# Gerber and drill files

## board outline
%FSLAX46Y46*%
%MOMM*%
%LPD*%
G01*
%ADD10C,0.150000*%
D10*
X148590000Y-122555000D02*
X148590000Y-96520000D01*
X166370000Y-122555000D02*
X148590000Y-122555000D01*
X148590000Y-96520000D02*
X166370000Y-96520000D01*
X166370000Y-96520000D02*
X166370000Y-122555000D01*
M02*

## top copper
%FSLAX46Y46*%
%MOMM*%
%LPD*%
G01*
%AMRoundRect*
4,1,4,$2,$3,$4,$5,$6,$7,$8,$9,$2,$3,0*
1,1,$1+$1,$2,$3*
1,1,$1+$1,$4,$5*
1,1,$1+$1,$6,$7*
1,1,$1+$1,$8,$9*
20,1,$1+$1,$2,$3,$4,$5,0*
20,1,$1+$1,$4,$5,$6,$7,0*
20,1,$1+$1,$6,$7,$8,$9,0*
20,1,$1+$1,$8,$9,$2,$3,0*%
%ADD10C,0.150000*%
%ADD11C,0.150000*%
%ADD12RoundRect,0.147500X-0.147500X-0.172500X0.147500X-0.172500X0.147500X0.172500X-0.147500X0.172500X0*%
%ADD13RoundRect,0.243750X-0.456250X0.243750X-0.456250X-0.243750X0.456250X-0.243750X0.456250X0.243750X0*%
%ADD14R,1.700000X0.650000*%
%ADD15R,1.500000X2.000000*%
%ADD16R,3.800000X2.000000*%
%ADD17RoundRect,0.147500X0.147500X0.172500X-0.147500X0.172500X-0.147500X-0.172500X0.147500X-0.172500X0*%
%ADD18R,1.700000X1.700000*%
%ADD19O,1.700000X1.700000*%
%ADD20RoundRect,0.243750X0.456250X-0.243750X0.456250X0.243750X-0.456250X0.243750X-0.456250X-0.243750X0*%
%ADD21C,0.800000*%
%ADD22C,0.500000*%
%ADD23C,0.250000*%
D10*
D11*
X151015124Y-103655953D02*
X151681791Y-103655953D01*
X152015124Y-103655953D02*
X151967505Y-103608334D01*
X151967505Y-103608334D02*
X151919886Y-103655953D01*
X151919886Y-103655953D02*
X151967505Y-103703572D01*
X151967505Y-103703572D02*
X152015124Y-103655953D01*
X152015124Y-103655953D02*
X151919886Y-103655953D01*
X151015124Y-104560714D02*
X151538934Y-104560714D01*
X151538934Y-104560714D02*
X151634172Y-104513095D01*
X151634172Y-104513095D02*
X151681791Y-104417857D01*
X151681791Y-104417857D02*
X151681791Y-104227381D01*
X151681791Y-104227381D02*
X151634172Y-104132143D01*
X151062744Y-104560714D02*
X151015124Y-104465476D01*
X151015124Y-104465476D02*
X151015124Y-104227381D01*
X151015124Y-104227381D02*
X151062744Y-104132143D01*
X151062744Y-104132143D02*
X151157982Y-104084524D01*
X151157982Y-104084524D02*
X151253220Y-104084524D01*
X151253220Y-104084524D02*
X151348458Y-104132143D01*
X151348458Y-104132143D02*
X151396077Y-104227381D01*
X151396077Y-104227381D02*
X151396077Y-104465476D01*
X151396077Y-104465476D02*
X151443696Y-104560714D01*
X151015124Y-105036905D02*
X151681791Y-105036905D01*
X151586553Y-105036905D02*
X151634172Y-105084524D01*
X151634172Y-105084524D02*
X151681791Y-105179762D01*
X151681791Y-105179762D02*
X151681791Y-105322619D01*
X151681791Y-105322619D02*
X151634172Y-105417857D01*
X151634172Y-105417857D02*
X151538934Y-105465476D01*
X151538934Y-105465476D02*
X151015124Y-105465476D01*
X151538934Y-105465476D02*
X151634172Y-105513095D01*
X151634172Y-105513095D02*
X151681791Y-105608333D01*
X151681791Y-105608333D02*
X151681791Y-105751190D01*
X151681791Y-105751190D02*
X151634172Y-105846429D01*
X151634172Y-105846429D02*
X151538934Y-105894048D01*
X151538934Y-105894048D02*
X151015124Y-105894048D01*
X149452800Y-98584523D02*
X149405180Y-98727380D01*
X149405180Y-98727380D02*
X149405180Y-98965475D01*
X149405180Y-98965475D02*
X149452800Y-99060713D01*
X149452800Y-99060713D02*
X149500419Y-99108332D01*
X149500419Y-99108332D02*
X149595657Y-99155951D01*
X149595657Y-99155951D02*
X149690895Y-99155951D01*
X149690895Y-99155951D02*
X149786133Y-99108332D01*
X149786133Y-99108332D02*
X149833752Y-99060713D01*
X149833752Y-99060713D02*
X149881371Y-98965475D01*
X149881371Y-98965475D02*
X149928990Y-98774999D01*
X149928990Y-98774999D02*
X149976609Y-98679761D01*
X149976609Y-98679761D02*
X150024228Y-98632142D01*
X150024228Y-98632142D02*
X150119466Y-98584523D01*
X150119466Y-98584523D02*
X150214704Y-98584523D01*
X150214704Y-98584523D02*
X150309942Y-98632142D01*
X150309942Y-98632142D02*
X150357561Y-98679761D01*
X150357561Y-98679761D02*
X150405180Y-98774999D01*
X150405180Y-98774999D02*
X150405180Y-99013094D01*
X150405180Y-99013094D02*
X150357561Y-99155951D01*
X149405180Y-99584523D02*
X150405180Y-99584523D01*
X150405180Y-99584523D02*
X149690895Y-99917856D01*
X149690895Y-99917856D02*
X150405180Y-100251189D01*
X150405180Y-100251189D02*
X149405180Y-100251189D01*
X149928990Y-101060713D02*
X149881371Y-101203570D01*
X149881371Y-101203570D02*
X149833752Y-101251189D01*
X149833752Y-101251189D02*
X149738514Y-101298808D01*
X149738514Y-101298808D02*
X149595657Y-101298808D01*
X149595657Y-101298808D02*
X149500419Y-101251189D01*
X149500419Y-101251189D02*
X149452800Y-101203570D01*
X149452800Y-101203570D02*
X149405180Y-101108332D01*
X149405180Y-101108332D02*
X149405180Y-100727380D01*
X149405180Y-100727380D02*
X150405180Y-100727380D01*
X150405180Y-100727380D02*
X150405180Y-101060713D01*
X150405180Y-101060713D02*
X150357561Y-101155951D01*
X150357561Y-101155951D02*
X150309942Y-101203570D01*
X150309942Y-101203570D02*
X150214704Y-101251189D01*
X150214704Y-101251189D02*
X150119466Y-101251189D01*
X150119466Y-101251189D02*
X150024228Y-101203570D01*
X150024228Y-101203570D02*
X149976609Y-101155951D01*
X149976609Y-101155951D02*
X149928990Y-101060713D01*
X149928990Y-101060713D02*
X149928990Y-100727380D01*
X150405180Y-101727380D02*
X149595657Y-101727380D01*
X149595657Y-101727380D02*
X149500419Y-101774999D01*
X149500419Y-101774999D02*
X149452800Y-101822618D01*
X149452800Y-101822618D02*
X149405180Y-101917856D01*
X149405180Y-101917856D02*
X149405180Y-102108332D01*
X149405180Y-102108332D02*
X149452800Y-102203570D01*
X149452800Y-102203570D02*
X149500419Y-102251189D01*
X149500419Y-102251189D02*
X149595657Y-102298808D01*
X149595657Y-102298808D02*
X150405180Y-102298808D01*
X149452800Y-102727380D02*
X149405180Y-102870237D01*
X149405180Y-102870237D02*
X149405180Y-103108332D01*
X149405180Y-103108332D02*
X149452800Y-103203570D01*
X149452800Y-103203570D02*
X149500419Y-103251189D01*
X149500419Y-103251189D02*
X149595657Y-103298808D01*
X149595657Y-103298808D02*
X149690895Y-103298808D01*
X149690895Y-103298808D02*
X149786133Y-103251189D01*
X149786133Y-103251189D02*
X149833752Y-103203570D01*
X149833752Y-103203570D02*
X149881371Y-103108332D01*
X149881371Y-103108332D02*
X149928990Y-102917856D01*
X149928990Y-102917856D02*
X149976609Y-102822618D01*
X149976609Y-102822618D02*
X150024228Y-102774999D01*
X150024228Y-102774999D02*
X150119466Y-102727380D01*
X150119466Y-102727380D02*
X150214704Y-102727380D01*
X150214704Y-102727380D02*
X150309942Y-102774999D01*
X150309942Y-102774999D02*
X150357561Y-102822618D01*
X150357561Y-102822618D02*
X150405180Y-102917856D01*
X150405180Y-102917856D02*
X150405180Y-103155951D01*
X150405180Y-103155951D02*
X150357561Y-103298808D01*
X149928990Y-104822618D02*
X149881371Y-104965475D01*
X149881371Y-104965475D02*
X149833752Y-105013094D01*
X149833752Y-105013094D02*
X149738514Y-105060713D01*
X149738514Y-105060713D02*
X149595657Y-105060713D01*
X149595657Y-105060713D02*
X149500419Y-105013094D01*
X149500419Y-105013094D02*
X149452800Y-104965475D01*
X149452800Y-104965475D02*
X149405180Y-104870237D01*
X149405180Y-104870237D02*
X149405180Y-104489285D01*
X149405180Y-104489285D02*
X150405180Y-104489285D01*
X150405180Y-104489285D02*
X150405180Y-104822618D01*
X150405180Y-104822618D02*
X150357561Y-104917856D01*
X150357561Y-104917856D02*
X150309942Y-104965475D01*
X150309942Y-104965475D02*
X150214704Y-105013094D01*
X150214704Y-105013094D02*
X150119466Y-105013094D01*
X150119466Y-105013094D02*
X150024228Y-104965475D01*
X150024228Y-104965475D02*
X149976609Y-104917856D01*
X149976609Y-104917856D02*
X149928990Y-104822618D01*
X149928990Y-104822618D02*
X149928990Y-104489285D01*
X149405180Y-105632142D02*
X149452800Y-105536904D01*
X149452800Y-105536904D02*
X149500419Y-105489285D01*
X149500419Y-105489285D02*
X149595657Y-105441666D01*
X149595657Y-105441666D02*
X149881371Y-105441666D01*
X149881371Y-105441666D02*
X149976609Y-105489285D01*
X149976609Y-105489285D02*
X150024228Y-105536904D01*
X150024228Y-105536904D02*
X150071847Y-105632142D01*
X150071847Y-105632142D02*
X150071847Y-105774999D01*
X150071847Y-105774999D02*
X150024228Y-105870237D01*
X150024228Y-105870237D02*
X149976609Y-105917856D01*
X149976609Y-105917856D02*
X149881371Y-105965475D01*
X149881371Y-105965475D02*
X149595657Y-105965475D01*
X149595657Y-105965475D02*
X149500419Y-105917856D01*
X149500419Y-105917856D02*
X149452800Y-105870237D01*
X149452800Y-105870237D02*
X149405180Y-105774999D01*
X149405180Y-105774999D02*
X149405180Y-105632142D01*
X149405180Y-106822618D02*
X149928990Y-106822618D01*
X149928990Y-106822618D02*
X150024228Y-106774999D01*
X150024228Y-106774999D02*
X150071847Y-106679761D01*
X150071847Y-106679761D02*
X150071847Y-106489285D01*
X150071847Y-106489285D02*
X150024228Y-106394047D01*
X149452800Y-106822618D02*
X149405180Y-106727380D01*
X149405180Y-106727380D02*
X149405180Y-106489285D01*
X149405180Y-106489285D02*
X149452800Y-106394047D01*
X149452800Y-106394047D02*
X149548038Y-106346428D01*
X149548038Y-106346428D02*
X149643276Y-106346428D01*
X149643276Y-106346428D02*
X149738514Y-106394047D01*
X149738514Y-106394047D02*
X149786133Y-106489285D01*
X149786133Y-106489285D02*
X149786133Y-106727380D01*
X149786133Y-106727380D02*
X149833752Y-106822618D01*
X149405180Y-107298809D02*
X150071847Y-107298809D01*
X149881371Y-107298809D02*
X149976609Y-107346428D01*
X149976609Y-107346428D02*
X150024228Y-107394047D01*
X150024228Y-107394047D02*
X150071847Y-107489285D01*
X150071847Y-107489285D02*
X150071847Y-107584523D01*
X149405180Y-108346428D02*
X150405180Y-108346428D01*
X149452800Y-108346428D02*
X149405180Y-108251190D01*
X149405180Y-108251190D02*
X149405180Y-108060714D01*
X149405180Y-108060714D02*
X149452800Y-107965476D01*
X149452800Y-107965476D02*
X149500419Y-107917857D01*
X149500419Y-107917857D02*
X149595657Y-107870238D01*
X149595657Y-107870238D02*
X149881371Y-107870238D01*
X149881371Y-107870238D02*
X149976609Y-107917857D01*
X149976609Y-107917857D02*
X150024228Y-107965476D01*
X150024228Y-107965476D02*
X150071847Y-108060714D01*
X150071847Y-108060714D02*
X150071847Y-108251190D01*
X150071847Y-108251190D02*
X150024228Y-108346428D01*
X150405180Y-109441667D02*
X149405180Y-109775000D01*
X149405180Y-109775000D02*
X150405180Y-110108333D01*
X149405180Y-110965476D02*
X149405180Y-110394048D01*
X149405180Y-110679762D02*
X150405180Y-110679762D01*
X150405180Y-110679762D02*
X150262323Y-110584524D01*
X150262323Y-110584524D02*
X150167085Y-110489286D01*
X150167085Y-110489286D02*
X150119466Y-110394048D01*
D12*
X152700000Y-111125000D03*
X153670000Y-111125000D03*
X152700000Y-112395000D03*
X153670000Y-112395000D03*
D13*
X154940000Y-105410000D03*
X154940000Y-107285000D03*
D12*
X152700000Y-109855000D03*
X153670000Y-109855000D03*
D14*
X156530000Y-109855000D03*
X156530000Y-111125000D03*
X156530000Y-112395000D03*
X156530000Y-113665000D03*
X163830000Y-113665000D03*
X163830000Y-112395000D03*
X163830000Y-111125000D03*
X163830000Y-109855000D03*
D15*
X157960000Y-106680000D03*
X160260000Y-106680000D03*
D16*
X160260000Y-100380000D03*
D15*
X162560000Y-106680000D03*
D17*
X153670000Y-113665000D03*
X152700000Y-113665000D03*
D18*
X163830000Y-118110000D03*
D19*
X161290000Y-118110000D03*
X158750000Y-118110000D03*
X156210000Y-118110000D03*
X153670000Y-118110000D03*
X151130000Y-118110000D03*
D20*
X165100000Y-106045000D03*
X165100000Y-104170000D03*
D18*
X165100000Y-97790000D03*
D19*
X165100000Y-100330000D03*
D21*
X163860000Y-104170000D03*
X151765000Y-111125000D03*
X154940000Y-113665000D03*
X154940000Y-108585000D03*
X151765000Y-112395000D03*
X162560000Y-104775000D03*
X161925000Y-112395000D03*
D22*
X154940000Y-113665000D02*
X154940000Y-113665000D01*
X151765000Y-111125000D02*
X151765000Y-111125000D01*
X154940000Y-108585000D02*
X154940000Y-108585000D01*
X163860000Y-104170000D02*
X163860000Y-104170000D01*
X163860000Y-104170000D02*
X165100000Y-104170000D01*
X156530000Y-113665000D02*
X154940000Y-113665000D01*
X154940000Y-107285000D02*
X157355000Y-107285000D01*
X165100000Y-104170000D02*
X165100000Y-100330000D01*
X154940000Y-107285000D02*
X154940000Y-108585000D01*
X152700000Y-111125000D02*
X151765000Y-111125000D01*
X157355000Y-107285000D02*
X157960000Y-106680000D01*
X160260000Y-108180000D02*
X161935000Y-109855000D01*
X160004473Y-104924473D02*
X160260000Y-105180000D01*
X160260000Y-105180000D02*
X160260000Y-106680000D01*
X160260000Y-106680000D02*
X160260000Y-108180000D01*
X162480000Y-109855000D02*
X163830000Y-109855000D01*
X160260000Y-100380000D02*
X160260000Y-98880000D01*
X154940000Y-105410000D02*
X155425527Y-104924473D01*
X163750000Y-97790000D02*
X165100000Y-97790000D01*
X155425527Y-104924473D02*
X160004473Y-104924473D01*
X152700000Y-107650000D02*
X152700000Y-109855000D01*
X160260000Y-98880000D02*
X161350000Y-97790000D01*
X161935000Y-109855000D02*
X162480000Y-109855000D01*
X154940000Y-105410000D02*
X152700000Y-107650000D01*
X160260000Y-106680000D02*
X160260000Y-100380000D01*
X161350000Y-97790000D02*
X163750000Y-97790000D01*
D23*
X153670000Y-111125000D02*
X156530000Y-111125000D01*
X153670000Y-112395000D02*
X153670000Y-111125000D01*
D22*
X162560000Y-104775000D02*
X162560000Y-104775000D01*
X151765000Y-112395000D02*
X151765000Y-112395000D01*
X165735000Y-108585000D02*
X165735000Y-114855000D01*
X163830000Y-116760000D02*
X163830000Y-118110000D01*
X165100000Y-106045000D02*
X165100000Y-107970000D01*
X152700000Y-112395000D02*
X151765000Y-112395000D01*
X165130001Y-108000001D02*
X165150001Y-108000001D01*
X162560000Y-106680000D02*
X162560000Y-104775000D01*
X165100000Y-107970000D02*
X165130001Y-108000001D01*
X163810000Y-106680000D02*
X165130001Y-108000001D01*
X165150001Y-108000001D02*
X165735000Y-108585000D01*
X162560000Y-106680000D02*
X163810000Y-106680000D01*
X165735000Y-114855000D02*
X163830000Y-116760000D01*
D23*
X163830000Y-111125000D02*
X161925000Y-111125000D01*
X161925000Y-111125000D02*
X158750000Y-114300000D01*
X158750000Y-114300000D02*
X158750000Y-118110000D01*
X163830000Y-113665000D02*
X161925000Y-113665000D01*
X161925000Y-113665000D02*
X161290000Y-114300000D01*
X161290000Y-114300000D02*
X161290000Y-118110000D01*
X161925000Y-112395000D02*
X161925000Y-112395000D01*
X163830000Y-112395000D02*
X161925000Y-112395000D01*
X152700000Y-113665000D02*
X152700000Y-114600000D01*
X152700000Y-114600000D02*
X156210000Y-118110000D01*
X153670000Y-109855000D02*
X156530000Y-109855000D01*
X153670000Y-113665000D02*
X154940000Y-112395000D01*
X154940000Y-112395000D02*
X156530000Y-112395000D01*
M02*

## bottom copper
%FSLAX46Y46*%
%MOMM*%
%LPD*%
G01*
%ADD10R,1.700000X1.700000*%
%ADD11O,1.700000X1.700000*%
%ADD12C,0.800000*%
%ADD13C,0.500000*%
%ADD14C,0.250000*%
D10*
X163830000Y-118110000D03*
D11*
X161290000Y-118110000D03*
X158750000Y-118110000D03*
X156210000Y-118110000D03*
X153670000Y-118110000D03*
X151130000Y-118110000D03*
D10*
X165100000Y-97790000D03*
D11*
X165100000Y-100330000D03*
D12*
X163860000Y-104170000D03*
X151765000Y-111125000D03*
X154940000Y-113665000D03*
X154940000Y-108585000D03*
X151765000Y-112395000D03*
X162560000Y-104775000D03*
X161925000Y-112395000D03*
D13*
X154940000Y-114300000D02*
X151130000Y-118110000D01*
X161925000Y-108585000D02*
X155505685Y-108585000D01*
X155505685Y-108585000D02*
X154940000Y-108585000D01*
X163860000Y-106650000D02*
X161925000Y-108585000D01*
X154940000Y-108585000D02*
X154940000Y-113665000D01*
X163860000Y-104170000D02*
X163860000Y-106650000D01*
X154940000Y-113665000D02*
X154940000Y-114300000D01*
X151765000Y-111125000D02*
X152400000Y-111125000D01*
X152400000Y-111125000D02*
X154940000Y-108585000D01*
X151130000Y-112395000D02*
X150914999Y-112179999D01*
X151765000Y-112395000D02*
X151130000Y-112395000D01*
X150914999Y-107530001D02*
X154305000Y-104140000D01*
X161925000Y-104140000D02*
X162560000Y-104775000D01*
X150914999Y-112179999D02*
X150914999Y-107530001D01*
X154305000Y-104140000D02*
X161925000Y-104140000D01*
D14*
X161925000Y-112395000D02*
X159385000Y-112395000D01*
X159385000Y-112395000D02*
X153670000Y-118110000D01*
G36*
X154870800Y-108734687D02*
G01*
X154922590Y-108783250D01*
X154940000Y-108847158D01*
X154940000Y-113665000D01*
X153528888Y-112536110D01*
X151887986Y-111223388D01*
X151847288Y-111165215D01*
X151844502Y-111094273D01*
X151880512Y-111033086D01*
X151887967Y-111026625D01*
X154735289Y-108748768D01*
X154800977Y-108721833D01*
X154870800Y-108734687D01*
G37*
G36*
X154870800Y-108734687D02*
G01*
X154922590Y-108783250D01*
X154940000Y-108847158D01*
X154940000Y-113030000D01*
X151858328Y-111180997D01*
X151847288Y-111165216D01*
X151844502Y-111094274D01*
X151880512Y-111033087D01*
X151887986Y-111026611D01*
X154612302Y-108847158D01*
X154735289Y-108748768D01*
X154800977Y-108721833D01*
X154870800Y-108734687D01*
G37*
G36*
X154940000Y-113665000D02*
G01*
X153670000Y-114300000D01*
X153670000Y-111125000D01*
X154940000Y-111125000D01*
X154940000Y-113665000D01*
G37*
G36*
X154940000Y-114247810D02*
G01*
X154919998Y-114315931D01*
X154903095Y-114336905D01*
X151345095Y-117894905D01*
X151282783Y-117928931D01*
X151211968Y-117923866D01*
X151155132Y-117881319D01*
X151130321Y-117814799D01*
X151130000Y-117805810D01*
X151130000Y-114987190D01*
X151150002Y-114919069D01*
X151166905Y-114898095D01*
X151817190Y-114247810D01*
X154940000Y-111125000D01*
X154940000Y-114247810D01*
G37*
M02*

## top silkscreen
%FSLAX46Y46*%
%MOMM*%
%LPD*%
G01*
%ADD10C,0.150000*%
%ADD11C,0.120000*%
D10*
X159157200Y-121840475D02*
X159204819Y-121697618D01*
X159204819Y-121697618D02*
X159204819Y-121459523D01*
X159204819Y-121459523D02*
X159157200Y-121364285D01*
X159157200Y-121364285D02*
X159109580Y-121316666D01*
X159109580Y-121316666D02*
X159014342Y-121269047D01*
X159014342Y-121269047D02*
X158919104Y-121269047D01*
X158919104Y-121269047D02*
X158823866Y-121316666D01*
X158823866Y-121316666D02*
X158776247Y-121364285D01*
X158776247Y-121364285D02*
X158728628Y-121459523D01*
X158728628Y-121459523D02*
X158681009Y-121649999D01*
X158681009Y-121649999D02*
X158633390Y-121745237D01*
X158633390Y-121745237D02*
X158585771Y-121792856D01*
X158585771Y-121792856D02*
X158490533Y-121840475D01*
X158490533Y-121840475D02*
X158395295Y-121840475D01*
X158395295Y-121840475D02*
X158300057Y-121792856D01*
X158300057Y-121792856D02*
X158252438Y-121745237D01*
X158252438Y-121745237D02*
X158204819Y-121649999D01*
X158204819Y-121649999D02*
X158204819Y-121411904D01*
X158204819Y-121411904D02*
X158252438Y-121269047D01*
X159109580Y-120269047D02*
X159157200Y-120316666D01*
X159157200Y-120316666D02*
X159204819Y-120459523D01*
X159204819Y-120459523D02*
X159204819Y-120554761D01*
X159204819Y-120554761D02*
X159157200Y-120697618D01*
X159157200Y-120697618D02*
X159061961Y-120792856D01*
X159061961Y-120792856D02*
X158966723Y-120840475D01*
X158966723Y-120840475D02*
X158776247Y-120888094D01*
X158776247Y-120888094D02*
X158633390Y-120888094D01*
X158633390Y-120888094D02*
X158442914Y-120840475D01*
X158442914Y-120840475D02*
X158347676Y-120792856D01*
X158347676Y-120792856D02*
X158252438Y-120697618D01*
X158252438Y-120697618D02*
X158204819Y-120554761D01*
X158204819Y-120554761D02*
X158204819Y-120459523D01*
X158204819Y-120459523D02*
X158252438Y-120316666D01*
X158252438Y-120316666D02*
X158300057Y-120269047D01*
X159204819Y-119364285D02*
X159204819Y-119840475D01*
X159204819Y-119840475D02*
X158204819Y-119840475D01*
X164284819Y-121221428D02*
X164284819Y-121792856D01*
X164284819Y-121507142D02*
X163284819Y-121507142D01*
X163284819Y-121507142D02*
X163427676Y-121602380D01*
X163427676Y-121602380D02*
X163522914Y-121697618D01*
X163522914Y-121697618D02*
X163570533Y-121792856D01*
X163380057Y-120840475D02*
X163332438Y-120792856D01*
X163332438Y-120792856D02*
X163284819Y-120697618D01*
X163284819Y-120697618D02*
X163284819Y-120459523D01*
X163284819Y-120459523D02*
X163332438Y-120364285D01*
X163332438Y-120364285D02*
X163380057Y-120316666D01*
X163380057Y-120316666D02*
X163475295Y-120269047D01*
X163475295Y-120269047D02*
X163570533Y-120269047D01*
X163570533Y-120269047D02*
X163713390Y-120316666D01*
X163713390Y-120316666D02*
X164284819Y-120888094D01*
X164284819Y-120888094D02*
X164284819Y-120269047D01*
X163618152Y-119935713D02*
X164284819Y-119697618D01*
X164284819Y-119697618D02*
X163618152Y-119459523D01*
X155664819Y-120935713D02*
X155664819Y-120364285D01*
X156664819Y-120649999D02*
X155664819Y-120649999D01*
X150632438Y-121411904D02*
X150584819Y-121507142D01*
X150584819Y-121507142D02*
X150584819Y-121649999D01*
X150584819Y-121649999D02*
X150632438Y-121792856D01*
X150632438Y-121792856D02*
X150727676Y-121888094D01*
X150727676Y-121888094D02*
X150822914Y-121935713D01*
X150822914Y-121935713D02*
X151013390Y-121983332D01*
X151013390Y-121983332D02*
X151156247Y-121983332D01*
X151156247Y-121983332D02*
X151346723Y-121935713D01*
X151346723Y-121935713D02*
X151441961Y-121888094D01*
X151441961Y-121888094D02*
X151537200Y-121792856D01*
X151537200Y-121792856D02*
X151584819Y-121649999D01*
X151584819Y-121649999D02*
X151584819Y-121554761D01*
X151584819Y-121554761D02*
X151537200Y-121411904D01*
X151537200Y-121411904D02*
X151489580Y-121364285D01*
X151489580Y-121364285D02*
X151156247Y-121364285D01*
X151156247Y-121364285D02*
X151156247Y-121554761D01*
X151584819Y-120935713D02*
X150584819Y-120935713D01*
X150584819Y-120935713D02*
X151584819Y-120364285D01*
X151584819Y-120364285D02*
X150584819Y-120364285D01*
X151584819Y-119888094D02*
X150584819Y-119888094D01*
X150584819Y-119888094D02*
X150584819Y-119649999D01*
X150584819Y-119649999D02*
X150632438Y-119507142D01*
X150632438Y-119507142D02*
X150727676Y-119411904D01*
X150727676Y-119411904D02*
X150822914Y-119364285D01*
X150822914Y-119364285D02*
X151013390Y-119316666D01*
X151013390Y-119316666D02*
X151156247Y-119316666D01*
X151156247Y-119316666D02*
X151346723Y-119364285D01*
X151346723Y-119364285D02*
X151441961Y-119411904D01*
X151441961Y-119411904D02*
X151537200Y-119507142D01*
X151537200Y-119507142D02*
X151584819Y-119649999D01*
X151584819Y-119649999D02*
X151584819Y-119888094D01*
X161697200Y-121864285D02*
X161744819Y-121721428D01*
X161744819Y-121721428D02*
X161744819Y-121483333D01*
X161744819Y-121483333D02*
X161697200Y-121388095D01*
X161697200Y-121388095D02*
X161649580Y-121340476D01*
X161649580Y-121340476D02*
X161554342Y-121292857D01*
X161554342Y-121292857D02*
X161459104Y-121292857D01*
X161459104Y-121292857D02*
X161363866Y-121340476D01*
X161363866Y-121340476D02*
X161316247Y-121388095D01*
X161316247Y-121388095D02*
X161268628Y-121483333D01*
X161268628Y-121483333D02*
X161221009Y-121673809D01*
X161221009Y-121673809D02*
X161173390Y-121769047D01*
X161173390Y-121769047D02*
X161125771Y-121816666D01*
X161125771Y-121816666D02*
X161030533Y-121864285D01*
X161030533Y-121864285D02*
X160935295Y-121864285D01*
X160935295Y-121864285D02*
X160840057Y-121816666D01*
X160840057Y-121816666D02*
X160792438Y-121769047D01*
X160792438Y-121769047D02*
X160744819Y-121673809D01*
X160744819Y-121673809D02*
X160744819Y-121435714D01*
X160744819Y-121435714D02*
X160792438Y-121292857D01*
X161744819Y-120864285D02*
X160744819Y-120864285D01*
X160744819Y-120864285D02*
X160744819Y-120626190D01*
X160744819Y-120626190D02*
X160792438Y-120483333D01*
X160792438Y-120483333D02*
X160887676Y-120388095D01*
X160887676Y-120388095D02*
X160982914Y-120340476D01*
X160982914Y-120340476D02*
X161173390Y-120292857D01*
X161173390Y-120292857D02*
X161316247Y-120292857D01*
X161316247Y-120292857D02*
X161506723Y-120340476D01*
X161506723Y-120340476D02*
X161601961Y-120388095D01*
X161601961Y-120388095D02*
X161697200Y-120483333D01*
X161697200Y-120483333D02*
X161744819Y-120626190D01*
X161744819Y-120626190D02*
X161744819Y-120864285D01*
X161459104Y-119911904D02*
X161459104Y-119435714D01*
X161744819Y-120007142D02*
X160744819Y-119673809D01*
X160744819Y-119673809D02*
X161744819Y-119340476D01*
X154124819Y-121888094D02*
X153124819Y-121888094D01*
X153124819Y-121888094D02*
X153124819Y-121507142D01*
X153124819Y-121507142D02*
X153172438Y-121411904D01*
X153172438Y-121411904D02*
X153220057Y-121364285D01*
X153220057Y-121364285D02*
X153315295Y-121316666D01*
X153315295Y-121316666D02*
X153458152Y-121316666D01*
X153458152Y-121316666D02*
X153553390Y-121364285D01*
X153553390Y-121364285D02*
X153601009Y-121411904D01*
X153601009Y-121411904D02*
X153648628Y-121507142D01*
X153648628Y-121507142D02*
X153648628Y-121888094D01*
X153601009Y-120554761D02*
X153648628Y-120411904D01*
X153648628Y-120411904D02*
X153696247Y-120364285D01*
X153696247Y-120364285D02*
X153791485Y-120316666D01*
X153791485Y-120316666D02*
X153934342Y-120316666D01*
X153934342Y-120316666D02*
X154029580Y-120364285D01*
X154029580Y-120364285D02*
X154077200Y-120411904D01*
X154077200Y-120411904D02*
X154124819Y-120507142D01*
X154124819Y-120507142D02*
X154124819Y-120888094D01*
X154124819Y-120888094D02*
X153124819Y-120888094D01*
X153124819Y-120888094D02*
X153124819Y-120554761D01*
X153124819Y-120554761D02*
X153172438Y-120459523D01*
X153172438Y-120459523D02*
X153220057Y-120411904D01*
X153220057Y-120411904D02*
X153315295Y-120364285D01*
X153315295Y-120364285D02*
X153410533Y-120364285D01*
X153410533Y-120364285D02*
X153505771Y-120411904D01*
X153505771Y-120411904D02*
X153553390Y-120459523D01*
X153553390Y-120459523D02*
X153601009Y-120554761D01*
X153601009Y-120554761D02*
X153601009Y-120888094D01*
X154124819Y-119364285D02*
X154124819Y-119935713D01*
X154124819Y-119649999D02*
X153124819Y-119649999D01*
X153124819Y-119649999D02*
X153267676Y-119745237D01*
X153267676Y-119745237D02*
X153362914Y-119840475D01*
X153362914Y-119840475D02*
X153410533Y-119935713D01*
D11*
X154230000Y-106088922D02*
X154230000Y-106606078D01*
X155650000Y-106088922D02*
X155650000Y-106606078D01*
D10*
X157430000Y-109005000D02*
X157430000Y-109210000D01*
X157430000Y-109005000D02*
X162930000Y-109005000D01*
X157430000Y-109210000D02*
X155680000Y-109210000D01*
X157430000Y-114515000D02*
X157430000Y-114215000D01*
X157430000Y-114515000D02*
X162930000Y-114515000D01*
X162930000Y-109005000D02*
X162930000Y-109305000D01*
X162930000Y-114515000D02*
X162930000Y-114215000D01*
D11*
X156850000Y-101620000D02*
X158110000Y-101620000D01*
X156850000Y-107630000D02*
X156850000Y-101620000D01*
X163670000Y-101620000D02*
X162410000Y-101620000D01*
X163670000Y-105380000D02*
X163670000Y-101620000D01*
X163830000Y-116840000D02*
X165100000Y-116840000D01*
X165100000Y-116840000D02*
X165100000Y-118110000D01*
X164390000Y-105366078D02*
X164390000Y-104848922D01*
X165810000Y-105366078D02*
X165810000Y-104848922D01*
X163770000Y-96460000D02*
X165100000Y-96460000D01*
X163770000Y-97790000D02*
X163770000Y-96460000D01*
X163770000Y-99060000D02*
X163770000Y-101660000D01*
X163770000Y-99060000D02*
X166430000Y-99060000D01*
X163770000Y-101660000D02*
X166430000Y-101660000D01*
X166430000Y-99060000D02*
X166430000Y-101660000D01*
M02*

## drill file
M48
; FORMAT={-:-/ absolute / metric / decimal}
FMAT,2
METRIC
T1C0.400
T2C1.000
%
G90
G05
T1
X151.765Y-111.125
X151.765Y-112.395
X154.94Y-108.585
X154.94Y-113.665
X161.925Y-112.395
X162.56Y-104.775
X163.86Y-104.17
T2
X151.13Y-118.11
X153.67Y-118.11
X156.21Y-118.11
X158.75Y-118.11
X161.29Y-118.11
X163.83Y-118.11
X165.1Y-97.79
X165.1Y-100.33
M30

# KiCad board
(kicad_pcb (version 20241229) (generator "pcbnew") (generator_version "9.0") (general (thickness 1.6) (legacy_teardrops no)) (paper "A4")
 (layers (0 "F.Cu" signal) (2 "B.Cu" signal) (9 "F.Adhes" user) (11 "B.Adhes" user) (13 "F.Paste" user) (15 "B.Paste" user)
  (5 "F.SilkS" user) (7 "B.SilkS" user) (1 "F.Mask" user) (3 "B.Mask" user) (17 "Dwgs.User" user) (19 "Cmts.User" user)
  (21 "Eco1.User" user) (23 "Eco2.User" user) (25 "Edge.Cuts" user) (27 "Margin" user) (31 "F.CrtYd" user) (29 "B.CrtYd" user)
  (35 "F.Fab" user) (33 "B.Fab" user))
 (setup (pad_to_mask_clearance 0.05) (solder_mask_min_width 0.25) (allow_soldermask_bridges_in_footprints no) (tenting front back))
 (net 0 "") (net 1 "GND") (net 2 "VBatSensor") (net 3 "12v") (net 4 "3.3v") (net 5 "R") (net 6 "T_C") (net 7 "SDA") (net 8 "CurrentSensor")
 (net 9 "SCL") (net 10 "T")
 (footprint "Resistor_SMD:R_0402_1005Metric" (layer "F.Cu") (at 153.185 111.125)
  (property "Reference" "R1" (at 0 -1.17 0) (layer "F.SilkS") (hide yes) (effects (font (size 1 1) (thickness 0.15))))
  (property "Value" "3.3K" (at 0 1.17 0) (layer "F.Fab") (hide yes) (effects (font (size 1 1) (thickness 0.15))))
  (pad "1" smd roundrect (at -0.485 0) (size 0.59 0.64) (layers "F.Cu" "F.Mask" "F.Paste") (roundrect_rratio 0.25) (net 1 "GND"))
  (pad "2" smd roundrect (at 0.485 0) (size 0.59 0.64) (layers "F.Cu" "F.Mask" "F.Paste") (roundrect_rratio 0.25) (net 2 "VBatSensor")))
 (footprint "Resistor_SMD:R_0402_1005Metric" (layer "F.Cu") (at 153.185 112.395)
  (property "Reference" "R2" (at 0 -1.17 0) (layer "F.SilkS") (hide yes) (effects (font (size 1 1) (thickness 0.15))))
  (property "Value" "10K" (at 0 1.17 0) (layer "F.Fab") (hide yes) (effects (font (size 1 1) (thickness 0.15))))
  (pad "1" smd roundrect (at -0.485 0) (size 0.59 0.64) (layers "F.Cu" "F.Mask" "F.Paste") (roundrect_rratio 0.25) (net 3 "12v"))
  (pad "2" smd roundrect (at 0.485 0) (size 0.59 0.64) (layers "F.Cu" "F.Mask" "F.Paste") (roundrect_rratio 0.25) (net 2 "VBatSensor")))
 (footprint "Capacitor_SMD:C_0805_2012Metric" (layer "F.Cu") (at 154.94 106.3475 -90)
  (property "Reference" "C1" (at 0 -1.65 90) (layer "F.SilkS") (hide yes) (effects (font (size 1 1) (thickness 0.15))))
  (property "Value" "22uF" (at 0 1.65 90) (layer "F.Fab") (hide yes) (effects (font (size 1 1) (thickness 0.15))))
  (fp_line (start -0.258578 0.71) (end 0.258578 0.71) (stroke (width 0.12) (type solid)) (layer "F.SilkS"))
  (fp_line (start -0.258578 -0.71) (end 0.258578 -0.71) (stroke (width 0.12) (type solid)) (layer "F.SilkS"))
  (pad "1" smd roundrect (at -0.9375 0 270) (size 0.975 1.4) (layers "F.Cu" "F.Mask" "F.Paste") (roundrect_rratio 0.25) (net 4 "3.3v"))
  (pad "2" smd roundrect (at 0.9375 0 270) (size 0.975 1.4) (layers "F.Cu" "F.Mask" "F.Paste") (roundrect_rratio 0.25) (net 1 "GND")))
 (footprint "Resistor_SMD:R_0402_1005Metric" (layer "F.Cu") (at 153.185 109.855)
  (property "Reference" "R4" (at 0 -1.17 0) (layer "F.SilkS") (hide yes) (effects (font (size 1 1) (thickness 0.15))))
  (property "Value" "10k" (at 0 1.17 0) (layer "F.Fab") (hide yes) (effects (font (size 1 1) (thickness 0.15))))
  (pad "1" smd roundrect (at -0.485 0) (size 0.59 0.64) (layers "F.Cu" "F.Mask" "F.Paste") (roundrect_rratio 0.25) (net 4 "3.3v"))
  (pad "2" smd roundrect (at 0.485 0) (size 0.59 0.64) (layers "F.Cu" "F.Mask" "F.Paste") (roundrect_rratio 0.25) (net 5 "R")))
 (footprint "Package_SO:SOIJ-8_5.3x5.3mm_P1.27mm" (layer "F.Cu") (at 160.18 111.76)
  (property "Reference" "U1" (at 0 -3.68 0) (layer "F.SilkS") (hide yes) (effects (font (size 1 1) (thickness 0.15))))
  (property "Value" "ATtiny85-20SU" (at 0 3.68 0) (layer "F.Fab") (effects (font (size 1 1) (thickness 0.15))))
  (fp_line (start -2.75 -2.755) (end -2.75 -2.55) (stroke (width 0.15) (type solid)) (layer "F.SilkS"))
  (fp_line (start -2.75 -2.755) (end 2.75 -2.755) (stroke (width 0.15) (type solid)) (layer "F.SilkS"))
  (fp_line (start -2.75 -2.55) (end -4.5 -2.55) (stroke (width 0.15) (type solid)) (layer "F.SilkS"))
  (fp_line (start -2.75 2.755) (end -2.75 2.455) (stroke (width 0.15) (type solid)) (layer "F.SilkS"))
  (fp_line (start -2.75 2.755) (end 2.75 2.755) (stroke (width 0.15) (type solid)) (layer "F.SilkS"))
  (fp_line (start 2.75 -2.755) (end 2.75 -2.455) (stroke (width 0.15) (type solid)) (layer "F.SilkS"))
  (fp_line (start 2.75 2.755) (end 2.75 2.455) (stroke (width 0.15) (type solid)) (layer "F.SilkS"))
  (pad "1" smd rect (at -3.65 -1.905) (size 1.7 0.65) (layers "F.Cu" "F.Mask" "F.Paste") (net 5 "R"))
  (pad "2" smd rect (at -3.65 -0.635) (size 1.7 0.65) (layers "F.Cu" "F.Mask" "F.Paste") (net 2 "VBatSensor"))
  (pad "3" smd rect (at -3.65 0.635) (size 1.7 0.65) (layers "F.Cu" "F.Mask" "F.Paste") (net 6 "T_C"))
  (pad "4" smd rect (at -3.65 1.905) (size 1.7 0.65) (layers "F.Cu" "F.Mask" "F.Paste") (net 1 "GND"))
  (pad "5" smd rect (at 3.65 1.905) (size 1.7 0.65) (layers "F.Cu" "F.Mask" "F.Paste") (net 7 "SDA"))
  (pad "6" smd rect (at 3.65 0.635) (size 1.7 0.65) (layers "F.Cu" "F.Mask" "F.Paste") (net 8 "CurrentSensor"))
  (pad "7" smd rect (at 3.65 -0.635) (size 1.7 0.65) (layers "F.Cu" "F.Mask" "F.Paste") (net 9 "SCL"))
  (pad "8" smd rect (at 3.65 -1.905) (size 1.7 0.65) (layers "F.Cu" "F.Mask" "F.Paste") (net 4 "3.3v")))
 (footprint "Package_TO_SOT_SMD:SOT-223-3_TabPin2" (layer "F.Cu") (at 160.26 103.53 90)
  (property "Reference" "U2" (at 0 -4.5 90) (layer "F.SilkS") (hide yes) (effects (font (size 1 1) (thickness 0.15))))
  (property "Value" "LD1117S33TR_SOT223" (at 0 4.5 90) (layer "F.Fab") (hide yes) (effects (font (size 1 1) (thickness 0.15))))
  (fp_line (start 1.91 -3.41) (end 1.91 -2.15) (stroke (width 0.12) (type solid)) (layer "F.SilkS"))
  (fp_line (start -4.1 -3.41) (end 1.91 -3.41) (stroke (width 0.12) (type solid)) (layer "F.SilkS"))
  (fp_line (start 1.91 3.41) (end 1.91 2.15) (stroke (width 0.12) (type solid)) (layer "F.SilkS"))
  (fp_line (start -1.85 3.41) (end 1.91 3.41) (stroke (width 0.12) (type solid)) (layer "F.SilkS"))
  (pad "1" smd rect (at -3.15 -2.3 90) (size 2 1.5) (layers "F.Cu" "F.Mask" "F.Paste") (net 1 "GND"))
  (pad "2" smd rect (at -3.15 0 90) (size 2 1.5) (layers "F.Cu" "F.Mask" "F.Paste") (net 4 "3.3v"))
  (pad "2" smd rect (at 3.15 0 90) (size 2 3.8) (layers "F.Cu" "F.Mask" "F.Paste") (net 4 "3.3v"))
  (pad "3" smd rect (at -3.15 2.3 90) (size 2 1.5) (layers "F.Cu" "F.Mask" "F.Paste") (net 3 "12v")))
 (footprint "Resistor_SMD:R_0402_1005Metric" (layer "F.Cu") (at 153.185 113.665 180)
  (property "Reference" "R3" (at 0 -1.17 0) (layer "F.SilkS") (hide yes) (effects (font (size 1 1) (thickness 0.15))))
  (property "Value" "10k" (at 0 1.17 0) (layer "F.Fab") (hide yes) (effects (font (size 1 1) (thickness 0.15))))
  (pad "1" smd roundrect (at -0.485 0 180) (size 0.59 0.64) (layers "F.Cu" "F.Mask" "F.Paste") (roundrect_rratio 0.25) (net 6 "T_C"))
  (pad "2" smd roundrect (at 0.485 0 180) (size 0.59 0.64) (layers "F.Cu" "F.Mask" "F.Paste") (roundrect_rratio 0.25) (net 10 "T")))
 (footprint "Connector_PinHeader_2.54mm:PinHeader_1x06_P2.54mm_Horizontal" (layer "F.Cu") (at 163.83 118.11 -90)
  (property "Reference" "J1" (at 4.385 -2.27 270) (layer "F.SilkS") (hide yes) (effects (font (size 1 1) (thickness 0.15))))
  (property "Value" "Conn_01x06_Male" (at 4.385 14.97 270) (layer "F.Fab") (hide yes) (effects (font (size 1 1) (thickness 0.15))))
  (fp_line (start -1.27 0) (end -1.27 -1.27) (stroke (width 0.12) (type solid)) (layer "F.SilkS"))
  (fp_line (start -1.27 -1.27) (end 0 -1.27) (stroke (width 0.12) (type solid)) (layer "F.SilkS"))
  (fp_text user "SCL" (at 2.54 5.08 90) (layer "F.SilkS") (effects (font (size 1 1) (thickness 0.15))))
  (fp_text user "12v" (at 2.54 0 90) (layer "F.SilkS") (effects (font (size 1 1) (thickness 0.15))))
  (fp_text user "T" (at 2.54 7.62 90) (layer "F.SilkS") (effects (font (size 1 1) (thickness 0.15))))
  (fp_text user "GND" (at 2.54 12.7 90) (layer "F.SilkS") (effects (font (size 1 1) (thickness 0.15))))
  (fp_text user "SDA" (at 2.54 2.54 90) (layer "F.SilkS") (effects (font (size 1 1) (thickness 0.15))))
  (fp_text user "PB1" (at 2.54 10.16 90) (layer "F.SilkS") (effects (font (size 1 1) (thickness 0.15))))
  (pad "1" thru_hole rect (at 0 0 270) (size 1.7 1.7) (drill 1) (layers "*.Cu" "*.Mask") (remove_unused_layers no) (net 3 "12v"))
  (pad "2" thru_hole oval (at 0 2.54 270) (size 1.7 1.7) (drill 1) (layers "*.Cu" "*.Mask") (remove_unused_layers no) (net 7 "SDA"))
  (pad "3" thru_hole oval (at 0 5.08 270) (size 1.7 1.7) (drill 1) (layers "*.Cu" "*.Mask") (remove_unused_layers no) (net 9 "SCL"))
  (pad "4" thru_hole oval (at 0 7.62 270) (size 1.7 1.7) (drill 1) (layers "*.Cu" "*.Mask") (remove_unused_layers no) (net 10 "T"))
  (pad "5" thru_hole oval (at 0 10.16 270) (size 1.7 1.7) (drill 1) (layers "*.Cu" "*.Mask") (remove_unused_layers no)
   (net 8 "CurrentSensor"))
  (pad "6" thru_hole oval (at 0 12.7 270) (size 1.7 1.7) (drill 1) (layers "*.Cu" "*.Mask") (remove_unused_layers no) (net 1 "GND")))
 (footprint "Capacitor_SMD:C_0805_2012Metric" (layer "F.Cu") (at 165.1 105.1075 90)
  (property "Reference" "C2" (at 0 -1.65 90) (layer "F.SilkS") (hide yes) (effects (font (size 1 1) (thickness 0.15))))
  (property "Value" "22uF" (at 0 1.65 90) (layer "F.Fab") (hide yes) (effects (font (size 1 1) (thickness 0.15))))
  (fp_line (start -0.258578 -0.71) (end 0.258578 -0.71) (stroke (width 0.12) (type solid)) (layer "F.SilkS"))
  (fp_line (start -0.258578 0.71) (end 0.258578 0.71) (stroke (width 0.12) (type solid)) (layer "F.SilkS"))
  (pad "1" smd roundrect (at -0.9375 0 90) (size 0.975 1.4) (layers "F.Cu" "F.Mask" "F.Paste") (roundrect_rratio 0.25) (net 3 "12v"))
  (pad "2" smd roundrect (at 0.9375 0 90) (size 0.975 1.4) (layers "F.Cu" "F.Mask" "F.Paste") (roundrect_rratio 0.25) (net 1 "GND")))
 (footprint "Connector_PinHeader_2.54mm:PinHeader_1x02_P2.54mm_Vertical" (layer "F.Cu") (at 165.1 97.79)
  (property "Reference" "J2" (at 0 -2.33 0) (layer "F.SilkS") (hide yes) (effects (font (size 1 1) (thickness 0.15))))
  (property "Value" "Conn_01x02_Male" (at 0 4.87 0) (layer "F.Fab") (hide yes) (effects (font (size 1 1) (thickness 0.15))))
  (fp_line (start -1.33 -1.33) (end 0 -1.33) (stroke (width 0.12) (type solid)) (layer "F.SilkS"))
  (fp_line (start -1.33 0) (end -1.33 -1.33) (stroke (width 0.12) (type solid)) (layer "F.SilkS"))
  (fp_line (start -1.33 1.27) (end -1.33 3.87) (stroke (width 0.12) (type solid)) (layer "F.SilkS"))
  (fp_line (start -1.33 1.27) (end 1.33 1.27) (stroke (width 0.12) (type solid)) (layer "F.SilkS"))
  (fp_line (start -1.33 3.87) (end 1.33 3.87) (stroke (width 0.12) (type solid)) (layer "F.SilkS"))
  (fp_line (start 1.33 1.27) (end 1.33 3.87) (stroke (width 0.12) (type solid)) (layer "F.SilkS"))
  (pad "1" thru_hole rect (at 0 0) (size 1.7 1.7) (drill 1) (layers "*.Cu" "*.Mask") (remove_unused_layers no) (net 4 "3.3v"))
  (pad "2" thru_hole oval (at 0 2.54) (size 1.7 1.7) (drill 1) (layers "*.Cu" "*.Mask") (remove_unused_layers no) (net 1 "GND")))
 (gr_line (start 148.59 122.555) (end 148.59 96.52) (stroke (width 0.15) (type solid)) (layer "Edge.Cuts"))
 (gr_line (start 166.37 122.555) (end 148.59 122.555) (stroke (width 0.15) (type solid)) (layer "Edge.Cuts"))
 (gr_line (start 148.59 96.52) (end 166.37 96.52) (stroke (width 0.15) (type solid)) (layer "Edge.Cuts"))
 (gr_line (start 166.37 96.52) (end 166.37 122.555) (stroke (width 0.15) (type solid)) (layer "Edge.Cuts"))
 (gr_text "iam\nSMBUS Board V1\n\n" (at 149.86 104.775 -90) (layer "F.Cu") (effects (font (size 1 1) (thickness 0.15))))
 (segment (start 154.94 113.665) (end 154.94 113.665) (width 0.5) (layer "F.Cu") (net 1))
 (segment (start 151.765 111.125) (end 151.765 111.125) (width 0.5) (layer "F.Cu") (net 1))
 (segment (start 154.94 108.585) (end 154.94 108.585) (width 0.5) (layer "F.Cu") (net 1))
 (segment (start 163.86 104.17) (end 163.86 104.17) (width 0.5) (layer "F.Cu") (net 1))
 (segment (start 163.86 104.17) (end 165.1 104.17) (width 0.5) (layer "F.Cu") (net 1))
 (segment (start 156.53 113.665) (end 154.94 113.665) (width 0.5) (layer "F.Cu") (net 1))
 (segment (start 154.94 107.285) (end 157.355 107.285) (width 0.5) (layer "F.Cu") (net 1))
 (segment (start 165.1 104.17) (end 165.1 100.33) (width 0.5) (layer "F.Cu") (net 1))
 (segment (start 154.94 107.285) (end 154.94 108.585) (width 0.5) (layer "F.Cu") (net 1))
 (segment (start 152.7 111.125) (end 151.765 111.125) (width 0.5) (layer "F.Cu") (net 1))
 (segment (start 157.355 107.285) (end 157.96 106.68) (width 0.5) (layer "F.Cu") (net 1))
 (via (at 163.86 104.17) (size 0.8) (drill 0.4) (layers "F.Cu" "B.Cu") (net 1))
 (via (at 151.765 111.125) (size 0.8) (drill 0.4) (layers "F.Cu" "B.Cu") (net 1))
 (via (at 154.94 113.665) (size 0.8) (drill 0.4) (layers "F.Cu" "B.Cu") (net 1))
 (via (at 154.94 108.585) (size 0.8) (drill 0.4) (layers "F.Cu" "B.Cu") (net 1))
 (segment (start 154.94 114.3) (end 151.13 118.11) (width 0.5) (layer "B.Cu") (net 1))
 (segment (start 161.925 108.585) (end 155.505685 108.585) (width 0.5) (layer "B.Cu") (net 1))
 (segment (start 155.505685 108.585) (end 154.94 108.585) (width 0.5) (layer "B.Cu") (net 1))
 (segment (start 163.86 106.65) (end 161.925 108.585) (width 0.5) (layer "B.Cu") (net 1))
 (segment (start 154.94 108.585) (end 154.94 113.665) (width 0.5) (layer "B.Cu") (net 1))
 (segment (start 163.86 104.17) (end 163.86 106.65) (width 0.5) (layer "B.Cu") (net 1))
 (segment (start 154.94 113.665) (end 154.94 114.3) (width 0.5) (layer "B.Cu") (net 1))
 (segment (start 151.765 111.125) (end 152.4 111.125) (width 0.5) (layer "B.Cu") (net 1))
 (segment (start 152.4 111.125) (end 154.94 108.585) (width 0.5) (layer "B.Cu") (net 1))
 (segment (start 160.26 108.18) (end 161.935 109.855) (width 0.5) (layer "F.Cu") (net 4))
 (segment (start 160.004473 104.924473) (end 160.26 105.18) (width 0.5) (layer "F.Cu") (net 4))
 (segment (start 160.26 105.18) (end 160.26 106.68) (width 0.5) (layer "F.Cu") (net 4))
 (segment (start 160.26 106.68) (end 160.26 108.18) (width 0.5) (layer "F.Cu") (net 4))
 (segment (start 162.48 109.855) (end 163.83 109.855) (width 0.5) (layer "F.Cu") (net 4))
 (segment (start 160.26 100.38) (end 160.26 98.88) (width 0.5) (layer "F.Cu") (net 4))
 (segment (start 154.94 105.41) (end 155.425527 104.924473) (width 0.5) (layer "F.Cu") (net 4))
 (segment (start 163.75 97.79) (end 165.1 97.79) (width 0.5) (layer "F.Cu") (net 4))
 (segment (start 155.425527 104.924473) (end 160.004473 104.924473) (width 0.5) (layer "F.Cu") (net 4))
 (segment (start 152.7 107.65) (end 152.7 109.855) (width 0.5) (layer "F.Cu") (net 4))
 (segment (start 160.26 98.88) (end 161.35 97.79) (width 0.5) (layer "F.Cu") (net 4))
 (segment (start 161.935 109.855) (end 162.48 109.855) (width 0.5) (layer "F.Cu") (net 4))
 (segment (start 154.94 105.41) (end 152.7 107.65) (width 0.5) (layer "F.Cu") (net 4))
 (segment (start 160.26 106.68) (end 160.26 100.38) (width 0.5) (layer "F.Cu") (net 4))
 (segment (start 161.35 97.79) (end 163.75 97.79) (width 0.5) (layer "F.Cu") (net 4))
 (segment (start 153.67 111.125) (end 156.53 111.125) (width 0.25) (layer "F.Cu") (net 2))
 (segment (start 153.67 112.395) (end 153.67 111.125) (width 0.25) (layer "F.Cu") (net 2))
 (segment (start 162.56 104.775) (end 162.56 104.775) (width 0.5) (layer "F.Cu") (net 3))
 (segment (start 151.765 112.395) (end 151.765 112.395) (width 0.5) (layer "F.Cu") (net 3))
 (segment (start 165.735 108.585) (end 165.735 114.855) (width 0.5) (layer "F.Cu") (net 3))
 (segment (start 163.83 116.76) (end 163.83 118.11) (width 0.5) (layer "F.Cu") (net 3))
 (segment (start 165.1 106.045) (end 165.1 107.97) (width 0.5) (layer "F.Cu") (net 3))
 (segment (start 152.7 112.395) (end 151.765 112.395) (width 0.5) (layer "F.Cu") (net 3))
 (segment (start 165.130001 108.000001) (end 165.150001 108.000001) (width 0.5) (layer "F.Cu") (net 3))
 (segment (start 162.56 106.68) (end 162.56 104.775) (width 0.5) (layer "F.Cu") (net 3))
 (segment (start 165.1 107.97) (end 165.130001 108.000001) (width 0.5) (layer "F.Cu") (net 3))
 (segment (start 163.81 106.68) (end 165.130001 108.000001) (width 0.5) (layer "F.Cu") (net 3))
 (segment (start 165.150001 108.000001) (end 165.735 108.585) (width 0.5) (layer "F.Cu") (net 3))
 (segment (start 162.56 106.68) (end 163.81 106.68) (width 0.5) (layer "F.Cu") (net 3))
 (segment (start 165.735 114.855) (end 163.83 116.76) (width 0.5) (layer "F.Cu") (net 3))
 (via (at 151.765 112.395) (size 0.8) (drill 0.4) (layers "F.Cu" "B.Cu") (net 3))
 (via (at 162.56 104.775) (size 0.8) (drill 0.4) (layers "F.Cu" "B.Cu") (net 3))
 (segment (start 151.13 112.395) (end 150.914999 112.179999) (width 0.5) (layer "B.Cu") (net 3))
 (segment (start 151.765 112.395) (end 151.13 112.395) (width 0.5) (layer "B.Cu") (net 3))
 (segment (start 150.914999 107.530001) (end 154.305 104.14) (width 0.5) (layer "B.Cu") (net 3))
 (segment (start 161.925 104.14) (end 162.56 104.775) (width 0.5) (layer "B.Cu") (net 3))
 (segment (start 150.914999 112.179999) (end 150.914999 107.530001) (width 0.5) (layer "B.Cu") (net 3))
 (segment (start 154.305 104.14) (end 161.925 104.14) (width 0.5) (layer "B.Cu") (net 3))
 (segment (start 163.83 111.125) (end 161.925 111.125) (width 0.25) (layer "F.Cu") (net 9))
 (segment (start 161.925 111.125) (end 158.75 114.3) (width 0.25) (layer "F.Cu") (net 9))
 (segment (start 158.75 114.3) (end 158.75 118.11) (width 0.25) (layer "F.Cu") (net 9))
 (segment (start 163.83 113.665) (end 161.925 113.665) (width 0.25) (layer "F.Cu") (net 7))
 (segment (start 161.925 113.665) (end 161.29 114.3) (width 0.25) (layer "F.Cu") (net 7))
 (segment (start 161.29 114.3) (end 161.29 118.11) (width 0.25) (layer "F.Cu") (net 7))
 (segment (start 161.925 112.395) (end 161.925 112.395) (width 0.25) (layer "F.Cu") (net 8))
 (segment (start 163.83 112.395) (end 161.925 112.395) (width 0.25) (layer "F.Cu") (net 8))
 (via (at 161.925 112.395) (size 0.8) (drill 0.4) (layers "F.Cu" "B.Cu") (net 8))
 (segment (start 161.925 112.395) (end 159.385 112.395) (width 0.25) (layer "B.Cu") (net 8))
 (segment (start 159.385 112.395) (end 153.67 118.11) (width 0.25) (layer "B.Cu") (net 8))
 (segment (start 152.7 113.665) (end 152.7 114.6) (width 0.25) (layer "F.Cu") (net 10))
 (segment (start 152.7 114.6) (end 156.21 118.11) (width 0.25) (layer "F.Cu") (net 10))
 (segment (start 153.67 109.855) (end 156.53 109.855) (width 0.25) (layer "F.Cu") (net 5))
 (segment (start 153.67 113.665) (end 154.94 112.395) (width 0.25) (layer "F.Cu") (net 6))
 (segment (start 154.94 112.395) (end 156.53 112.395) (width 0.25) (layer "F.Cu") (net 6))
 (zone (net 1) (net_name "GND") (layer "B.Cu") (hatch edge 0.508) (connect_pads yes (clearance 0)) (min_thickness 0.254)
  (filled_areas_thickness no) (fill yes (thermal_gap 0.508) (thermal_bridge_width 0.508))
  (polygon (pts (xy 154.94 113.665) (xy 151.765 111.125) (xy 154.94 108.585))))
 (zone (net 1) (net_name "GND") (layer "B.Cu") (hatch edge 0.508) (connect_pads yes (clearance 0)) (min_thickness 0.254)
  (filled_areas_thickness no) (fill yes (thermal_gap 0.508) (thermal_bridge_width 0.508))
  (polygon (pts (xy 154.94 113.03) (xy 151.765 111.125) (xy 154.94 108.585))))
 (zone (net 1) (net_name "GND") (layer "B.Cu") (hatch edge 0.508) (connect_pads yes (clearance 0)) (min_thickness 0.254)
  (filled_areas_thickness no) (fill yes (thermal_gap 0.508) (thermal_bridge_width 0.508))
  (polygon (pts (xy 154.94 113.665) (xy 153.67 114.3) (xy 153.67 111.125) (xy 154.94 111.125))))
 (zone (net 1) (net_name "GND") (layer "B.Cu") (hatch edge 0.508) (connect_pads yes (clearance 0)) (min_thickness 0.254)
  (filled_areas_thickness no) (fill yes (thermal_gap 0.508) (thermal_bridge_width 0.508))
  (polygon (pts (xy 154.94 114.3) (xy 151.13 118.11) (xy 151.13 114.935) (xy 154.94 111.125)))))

